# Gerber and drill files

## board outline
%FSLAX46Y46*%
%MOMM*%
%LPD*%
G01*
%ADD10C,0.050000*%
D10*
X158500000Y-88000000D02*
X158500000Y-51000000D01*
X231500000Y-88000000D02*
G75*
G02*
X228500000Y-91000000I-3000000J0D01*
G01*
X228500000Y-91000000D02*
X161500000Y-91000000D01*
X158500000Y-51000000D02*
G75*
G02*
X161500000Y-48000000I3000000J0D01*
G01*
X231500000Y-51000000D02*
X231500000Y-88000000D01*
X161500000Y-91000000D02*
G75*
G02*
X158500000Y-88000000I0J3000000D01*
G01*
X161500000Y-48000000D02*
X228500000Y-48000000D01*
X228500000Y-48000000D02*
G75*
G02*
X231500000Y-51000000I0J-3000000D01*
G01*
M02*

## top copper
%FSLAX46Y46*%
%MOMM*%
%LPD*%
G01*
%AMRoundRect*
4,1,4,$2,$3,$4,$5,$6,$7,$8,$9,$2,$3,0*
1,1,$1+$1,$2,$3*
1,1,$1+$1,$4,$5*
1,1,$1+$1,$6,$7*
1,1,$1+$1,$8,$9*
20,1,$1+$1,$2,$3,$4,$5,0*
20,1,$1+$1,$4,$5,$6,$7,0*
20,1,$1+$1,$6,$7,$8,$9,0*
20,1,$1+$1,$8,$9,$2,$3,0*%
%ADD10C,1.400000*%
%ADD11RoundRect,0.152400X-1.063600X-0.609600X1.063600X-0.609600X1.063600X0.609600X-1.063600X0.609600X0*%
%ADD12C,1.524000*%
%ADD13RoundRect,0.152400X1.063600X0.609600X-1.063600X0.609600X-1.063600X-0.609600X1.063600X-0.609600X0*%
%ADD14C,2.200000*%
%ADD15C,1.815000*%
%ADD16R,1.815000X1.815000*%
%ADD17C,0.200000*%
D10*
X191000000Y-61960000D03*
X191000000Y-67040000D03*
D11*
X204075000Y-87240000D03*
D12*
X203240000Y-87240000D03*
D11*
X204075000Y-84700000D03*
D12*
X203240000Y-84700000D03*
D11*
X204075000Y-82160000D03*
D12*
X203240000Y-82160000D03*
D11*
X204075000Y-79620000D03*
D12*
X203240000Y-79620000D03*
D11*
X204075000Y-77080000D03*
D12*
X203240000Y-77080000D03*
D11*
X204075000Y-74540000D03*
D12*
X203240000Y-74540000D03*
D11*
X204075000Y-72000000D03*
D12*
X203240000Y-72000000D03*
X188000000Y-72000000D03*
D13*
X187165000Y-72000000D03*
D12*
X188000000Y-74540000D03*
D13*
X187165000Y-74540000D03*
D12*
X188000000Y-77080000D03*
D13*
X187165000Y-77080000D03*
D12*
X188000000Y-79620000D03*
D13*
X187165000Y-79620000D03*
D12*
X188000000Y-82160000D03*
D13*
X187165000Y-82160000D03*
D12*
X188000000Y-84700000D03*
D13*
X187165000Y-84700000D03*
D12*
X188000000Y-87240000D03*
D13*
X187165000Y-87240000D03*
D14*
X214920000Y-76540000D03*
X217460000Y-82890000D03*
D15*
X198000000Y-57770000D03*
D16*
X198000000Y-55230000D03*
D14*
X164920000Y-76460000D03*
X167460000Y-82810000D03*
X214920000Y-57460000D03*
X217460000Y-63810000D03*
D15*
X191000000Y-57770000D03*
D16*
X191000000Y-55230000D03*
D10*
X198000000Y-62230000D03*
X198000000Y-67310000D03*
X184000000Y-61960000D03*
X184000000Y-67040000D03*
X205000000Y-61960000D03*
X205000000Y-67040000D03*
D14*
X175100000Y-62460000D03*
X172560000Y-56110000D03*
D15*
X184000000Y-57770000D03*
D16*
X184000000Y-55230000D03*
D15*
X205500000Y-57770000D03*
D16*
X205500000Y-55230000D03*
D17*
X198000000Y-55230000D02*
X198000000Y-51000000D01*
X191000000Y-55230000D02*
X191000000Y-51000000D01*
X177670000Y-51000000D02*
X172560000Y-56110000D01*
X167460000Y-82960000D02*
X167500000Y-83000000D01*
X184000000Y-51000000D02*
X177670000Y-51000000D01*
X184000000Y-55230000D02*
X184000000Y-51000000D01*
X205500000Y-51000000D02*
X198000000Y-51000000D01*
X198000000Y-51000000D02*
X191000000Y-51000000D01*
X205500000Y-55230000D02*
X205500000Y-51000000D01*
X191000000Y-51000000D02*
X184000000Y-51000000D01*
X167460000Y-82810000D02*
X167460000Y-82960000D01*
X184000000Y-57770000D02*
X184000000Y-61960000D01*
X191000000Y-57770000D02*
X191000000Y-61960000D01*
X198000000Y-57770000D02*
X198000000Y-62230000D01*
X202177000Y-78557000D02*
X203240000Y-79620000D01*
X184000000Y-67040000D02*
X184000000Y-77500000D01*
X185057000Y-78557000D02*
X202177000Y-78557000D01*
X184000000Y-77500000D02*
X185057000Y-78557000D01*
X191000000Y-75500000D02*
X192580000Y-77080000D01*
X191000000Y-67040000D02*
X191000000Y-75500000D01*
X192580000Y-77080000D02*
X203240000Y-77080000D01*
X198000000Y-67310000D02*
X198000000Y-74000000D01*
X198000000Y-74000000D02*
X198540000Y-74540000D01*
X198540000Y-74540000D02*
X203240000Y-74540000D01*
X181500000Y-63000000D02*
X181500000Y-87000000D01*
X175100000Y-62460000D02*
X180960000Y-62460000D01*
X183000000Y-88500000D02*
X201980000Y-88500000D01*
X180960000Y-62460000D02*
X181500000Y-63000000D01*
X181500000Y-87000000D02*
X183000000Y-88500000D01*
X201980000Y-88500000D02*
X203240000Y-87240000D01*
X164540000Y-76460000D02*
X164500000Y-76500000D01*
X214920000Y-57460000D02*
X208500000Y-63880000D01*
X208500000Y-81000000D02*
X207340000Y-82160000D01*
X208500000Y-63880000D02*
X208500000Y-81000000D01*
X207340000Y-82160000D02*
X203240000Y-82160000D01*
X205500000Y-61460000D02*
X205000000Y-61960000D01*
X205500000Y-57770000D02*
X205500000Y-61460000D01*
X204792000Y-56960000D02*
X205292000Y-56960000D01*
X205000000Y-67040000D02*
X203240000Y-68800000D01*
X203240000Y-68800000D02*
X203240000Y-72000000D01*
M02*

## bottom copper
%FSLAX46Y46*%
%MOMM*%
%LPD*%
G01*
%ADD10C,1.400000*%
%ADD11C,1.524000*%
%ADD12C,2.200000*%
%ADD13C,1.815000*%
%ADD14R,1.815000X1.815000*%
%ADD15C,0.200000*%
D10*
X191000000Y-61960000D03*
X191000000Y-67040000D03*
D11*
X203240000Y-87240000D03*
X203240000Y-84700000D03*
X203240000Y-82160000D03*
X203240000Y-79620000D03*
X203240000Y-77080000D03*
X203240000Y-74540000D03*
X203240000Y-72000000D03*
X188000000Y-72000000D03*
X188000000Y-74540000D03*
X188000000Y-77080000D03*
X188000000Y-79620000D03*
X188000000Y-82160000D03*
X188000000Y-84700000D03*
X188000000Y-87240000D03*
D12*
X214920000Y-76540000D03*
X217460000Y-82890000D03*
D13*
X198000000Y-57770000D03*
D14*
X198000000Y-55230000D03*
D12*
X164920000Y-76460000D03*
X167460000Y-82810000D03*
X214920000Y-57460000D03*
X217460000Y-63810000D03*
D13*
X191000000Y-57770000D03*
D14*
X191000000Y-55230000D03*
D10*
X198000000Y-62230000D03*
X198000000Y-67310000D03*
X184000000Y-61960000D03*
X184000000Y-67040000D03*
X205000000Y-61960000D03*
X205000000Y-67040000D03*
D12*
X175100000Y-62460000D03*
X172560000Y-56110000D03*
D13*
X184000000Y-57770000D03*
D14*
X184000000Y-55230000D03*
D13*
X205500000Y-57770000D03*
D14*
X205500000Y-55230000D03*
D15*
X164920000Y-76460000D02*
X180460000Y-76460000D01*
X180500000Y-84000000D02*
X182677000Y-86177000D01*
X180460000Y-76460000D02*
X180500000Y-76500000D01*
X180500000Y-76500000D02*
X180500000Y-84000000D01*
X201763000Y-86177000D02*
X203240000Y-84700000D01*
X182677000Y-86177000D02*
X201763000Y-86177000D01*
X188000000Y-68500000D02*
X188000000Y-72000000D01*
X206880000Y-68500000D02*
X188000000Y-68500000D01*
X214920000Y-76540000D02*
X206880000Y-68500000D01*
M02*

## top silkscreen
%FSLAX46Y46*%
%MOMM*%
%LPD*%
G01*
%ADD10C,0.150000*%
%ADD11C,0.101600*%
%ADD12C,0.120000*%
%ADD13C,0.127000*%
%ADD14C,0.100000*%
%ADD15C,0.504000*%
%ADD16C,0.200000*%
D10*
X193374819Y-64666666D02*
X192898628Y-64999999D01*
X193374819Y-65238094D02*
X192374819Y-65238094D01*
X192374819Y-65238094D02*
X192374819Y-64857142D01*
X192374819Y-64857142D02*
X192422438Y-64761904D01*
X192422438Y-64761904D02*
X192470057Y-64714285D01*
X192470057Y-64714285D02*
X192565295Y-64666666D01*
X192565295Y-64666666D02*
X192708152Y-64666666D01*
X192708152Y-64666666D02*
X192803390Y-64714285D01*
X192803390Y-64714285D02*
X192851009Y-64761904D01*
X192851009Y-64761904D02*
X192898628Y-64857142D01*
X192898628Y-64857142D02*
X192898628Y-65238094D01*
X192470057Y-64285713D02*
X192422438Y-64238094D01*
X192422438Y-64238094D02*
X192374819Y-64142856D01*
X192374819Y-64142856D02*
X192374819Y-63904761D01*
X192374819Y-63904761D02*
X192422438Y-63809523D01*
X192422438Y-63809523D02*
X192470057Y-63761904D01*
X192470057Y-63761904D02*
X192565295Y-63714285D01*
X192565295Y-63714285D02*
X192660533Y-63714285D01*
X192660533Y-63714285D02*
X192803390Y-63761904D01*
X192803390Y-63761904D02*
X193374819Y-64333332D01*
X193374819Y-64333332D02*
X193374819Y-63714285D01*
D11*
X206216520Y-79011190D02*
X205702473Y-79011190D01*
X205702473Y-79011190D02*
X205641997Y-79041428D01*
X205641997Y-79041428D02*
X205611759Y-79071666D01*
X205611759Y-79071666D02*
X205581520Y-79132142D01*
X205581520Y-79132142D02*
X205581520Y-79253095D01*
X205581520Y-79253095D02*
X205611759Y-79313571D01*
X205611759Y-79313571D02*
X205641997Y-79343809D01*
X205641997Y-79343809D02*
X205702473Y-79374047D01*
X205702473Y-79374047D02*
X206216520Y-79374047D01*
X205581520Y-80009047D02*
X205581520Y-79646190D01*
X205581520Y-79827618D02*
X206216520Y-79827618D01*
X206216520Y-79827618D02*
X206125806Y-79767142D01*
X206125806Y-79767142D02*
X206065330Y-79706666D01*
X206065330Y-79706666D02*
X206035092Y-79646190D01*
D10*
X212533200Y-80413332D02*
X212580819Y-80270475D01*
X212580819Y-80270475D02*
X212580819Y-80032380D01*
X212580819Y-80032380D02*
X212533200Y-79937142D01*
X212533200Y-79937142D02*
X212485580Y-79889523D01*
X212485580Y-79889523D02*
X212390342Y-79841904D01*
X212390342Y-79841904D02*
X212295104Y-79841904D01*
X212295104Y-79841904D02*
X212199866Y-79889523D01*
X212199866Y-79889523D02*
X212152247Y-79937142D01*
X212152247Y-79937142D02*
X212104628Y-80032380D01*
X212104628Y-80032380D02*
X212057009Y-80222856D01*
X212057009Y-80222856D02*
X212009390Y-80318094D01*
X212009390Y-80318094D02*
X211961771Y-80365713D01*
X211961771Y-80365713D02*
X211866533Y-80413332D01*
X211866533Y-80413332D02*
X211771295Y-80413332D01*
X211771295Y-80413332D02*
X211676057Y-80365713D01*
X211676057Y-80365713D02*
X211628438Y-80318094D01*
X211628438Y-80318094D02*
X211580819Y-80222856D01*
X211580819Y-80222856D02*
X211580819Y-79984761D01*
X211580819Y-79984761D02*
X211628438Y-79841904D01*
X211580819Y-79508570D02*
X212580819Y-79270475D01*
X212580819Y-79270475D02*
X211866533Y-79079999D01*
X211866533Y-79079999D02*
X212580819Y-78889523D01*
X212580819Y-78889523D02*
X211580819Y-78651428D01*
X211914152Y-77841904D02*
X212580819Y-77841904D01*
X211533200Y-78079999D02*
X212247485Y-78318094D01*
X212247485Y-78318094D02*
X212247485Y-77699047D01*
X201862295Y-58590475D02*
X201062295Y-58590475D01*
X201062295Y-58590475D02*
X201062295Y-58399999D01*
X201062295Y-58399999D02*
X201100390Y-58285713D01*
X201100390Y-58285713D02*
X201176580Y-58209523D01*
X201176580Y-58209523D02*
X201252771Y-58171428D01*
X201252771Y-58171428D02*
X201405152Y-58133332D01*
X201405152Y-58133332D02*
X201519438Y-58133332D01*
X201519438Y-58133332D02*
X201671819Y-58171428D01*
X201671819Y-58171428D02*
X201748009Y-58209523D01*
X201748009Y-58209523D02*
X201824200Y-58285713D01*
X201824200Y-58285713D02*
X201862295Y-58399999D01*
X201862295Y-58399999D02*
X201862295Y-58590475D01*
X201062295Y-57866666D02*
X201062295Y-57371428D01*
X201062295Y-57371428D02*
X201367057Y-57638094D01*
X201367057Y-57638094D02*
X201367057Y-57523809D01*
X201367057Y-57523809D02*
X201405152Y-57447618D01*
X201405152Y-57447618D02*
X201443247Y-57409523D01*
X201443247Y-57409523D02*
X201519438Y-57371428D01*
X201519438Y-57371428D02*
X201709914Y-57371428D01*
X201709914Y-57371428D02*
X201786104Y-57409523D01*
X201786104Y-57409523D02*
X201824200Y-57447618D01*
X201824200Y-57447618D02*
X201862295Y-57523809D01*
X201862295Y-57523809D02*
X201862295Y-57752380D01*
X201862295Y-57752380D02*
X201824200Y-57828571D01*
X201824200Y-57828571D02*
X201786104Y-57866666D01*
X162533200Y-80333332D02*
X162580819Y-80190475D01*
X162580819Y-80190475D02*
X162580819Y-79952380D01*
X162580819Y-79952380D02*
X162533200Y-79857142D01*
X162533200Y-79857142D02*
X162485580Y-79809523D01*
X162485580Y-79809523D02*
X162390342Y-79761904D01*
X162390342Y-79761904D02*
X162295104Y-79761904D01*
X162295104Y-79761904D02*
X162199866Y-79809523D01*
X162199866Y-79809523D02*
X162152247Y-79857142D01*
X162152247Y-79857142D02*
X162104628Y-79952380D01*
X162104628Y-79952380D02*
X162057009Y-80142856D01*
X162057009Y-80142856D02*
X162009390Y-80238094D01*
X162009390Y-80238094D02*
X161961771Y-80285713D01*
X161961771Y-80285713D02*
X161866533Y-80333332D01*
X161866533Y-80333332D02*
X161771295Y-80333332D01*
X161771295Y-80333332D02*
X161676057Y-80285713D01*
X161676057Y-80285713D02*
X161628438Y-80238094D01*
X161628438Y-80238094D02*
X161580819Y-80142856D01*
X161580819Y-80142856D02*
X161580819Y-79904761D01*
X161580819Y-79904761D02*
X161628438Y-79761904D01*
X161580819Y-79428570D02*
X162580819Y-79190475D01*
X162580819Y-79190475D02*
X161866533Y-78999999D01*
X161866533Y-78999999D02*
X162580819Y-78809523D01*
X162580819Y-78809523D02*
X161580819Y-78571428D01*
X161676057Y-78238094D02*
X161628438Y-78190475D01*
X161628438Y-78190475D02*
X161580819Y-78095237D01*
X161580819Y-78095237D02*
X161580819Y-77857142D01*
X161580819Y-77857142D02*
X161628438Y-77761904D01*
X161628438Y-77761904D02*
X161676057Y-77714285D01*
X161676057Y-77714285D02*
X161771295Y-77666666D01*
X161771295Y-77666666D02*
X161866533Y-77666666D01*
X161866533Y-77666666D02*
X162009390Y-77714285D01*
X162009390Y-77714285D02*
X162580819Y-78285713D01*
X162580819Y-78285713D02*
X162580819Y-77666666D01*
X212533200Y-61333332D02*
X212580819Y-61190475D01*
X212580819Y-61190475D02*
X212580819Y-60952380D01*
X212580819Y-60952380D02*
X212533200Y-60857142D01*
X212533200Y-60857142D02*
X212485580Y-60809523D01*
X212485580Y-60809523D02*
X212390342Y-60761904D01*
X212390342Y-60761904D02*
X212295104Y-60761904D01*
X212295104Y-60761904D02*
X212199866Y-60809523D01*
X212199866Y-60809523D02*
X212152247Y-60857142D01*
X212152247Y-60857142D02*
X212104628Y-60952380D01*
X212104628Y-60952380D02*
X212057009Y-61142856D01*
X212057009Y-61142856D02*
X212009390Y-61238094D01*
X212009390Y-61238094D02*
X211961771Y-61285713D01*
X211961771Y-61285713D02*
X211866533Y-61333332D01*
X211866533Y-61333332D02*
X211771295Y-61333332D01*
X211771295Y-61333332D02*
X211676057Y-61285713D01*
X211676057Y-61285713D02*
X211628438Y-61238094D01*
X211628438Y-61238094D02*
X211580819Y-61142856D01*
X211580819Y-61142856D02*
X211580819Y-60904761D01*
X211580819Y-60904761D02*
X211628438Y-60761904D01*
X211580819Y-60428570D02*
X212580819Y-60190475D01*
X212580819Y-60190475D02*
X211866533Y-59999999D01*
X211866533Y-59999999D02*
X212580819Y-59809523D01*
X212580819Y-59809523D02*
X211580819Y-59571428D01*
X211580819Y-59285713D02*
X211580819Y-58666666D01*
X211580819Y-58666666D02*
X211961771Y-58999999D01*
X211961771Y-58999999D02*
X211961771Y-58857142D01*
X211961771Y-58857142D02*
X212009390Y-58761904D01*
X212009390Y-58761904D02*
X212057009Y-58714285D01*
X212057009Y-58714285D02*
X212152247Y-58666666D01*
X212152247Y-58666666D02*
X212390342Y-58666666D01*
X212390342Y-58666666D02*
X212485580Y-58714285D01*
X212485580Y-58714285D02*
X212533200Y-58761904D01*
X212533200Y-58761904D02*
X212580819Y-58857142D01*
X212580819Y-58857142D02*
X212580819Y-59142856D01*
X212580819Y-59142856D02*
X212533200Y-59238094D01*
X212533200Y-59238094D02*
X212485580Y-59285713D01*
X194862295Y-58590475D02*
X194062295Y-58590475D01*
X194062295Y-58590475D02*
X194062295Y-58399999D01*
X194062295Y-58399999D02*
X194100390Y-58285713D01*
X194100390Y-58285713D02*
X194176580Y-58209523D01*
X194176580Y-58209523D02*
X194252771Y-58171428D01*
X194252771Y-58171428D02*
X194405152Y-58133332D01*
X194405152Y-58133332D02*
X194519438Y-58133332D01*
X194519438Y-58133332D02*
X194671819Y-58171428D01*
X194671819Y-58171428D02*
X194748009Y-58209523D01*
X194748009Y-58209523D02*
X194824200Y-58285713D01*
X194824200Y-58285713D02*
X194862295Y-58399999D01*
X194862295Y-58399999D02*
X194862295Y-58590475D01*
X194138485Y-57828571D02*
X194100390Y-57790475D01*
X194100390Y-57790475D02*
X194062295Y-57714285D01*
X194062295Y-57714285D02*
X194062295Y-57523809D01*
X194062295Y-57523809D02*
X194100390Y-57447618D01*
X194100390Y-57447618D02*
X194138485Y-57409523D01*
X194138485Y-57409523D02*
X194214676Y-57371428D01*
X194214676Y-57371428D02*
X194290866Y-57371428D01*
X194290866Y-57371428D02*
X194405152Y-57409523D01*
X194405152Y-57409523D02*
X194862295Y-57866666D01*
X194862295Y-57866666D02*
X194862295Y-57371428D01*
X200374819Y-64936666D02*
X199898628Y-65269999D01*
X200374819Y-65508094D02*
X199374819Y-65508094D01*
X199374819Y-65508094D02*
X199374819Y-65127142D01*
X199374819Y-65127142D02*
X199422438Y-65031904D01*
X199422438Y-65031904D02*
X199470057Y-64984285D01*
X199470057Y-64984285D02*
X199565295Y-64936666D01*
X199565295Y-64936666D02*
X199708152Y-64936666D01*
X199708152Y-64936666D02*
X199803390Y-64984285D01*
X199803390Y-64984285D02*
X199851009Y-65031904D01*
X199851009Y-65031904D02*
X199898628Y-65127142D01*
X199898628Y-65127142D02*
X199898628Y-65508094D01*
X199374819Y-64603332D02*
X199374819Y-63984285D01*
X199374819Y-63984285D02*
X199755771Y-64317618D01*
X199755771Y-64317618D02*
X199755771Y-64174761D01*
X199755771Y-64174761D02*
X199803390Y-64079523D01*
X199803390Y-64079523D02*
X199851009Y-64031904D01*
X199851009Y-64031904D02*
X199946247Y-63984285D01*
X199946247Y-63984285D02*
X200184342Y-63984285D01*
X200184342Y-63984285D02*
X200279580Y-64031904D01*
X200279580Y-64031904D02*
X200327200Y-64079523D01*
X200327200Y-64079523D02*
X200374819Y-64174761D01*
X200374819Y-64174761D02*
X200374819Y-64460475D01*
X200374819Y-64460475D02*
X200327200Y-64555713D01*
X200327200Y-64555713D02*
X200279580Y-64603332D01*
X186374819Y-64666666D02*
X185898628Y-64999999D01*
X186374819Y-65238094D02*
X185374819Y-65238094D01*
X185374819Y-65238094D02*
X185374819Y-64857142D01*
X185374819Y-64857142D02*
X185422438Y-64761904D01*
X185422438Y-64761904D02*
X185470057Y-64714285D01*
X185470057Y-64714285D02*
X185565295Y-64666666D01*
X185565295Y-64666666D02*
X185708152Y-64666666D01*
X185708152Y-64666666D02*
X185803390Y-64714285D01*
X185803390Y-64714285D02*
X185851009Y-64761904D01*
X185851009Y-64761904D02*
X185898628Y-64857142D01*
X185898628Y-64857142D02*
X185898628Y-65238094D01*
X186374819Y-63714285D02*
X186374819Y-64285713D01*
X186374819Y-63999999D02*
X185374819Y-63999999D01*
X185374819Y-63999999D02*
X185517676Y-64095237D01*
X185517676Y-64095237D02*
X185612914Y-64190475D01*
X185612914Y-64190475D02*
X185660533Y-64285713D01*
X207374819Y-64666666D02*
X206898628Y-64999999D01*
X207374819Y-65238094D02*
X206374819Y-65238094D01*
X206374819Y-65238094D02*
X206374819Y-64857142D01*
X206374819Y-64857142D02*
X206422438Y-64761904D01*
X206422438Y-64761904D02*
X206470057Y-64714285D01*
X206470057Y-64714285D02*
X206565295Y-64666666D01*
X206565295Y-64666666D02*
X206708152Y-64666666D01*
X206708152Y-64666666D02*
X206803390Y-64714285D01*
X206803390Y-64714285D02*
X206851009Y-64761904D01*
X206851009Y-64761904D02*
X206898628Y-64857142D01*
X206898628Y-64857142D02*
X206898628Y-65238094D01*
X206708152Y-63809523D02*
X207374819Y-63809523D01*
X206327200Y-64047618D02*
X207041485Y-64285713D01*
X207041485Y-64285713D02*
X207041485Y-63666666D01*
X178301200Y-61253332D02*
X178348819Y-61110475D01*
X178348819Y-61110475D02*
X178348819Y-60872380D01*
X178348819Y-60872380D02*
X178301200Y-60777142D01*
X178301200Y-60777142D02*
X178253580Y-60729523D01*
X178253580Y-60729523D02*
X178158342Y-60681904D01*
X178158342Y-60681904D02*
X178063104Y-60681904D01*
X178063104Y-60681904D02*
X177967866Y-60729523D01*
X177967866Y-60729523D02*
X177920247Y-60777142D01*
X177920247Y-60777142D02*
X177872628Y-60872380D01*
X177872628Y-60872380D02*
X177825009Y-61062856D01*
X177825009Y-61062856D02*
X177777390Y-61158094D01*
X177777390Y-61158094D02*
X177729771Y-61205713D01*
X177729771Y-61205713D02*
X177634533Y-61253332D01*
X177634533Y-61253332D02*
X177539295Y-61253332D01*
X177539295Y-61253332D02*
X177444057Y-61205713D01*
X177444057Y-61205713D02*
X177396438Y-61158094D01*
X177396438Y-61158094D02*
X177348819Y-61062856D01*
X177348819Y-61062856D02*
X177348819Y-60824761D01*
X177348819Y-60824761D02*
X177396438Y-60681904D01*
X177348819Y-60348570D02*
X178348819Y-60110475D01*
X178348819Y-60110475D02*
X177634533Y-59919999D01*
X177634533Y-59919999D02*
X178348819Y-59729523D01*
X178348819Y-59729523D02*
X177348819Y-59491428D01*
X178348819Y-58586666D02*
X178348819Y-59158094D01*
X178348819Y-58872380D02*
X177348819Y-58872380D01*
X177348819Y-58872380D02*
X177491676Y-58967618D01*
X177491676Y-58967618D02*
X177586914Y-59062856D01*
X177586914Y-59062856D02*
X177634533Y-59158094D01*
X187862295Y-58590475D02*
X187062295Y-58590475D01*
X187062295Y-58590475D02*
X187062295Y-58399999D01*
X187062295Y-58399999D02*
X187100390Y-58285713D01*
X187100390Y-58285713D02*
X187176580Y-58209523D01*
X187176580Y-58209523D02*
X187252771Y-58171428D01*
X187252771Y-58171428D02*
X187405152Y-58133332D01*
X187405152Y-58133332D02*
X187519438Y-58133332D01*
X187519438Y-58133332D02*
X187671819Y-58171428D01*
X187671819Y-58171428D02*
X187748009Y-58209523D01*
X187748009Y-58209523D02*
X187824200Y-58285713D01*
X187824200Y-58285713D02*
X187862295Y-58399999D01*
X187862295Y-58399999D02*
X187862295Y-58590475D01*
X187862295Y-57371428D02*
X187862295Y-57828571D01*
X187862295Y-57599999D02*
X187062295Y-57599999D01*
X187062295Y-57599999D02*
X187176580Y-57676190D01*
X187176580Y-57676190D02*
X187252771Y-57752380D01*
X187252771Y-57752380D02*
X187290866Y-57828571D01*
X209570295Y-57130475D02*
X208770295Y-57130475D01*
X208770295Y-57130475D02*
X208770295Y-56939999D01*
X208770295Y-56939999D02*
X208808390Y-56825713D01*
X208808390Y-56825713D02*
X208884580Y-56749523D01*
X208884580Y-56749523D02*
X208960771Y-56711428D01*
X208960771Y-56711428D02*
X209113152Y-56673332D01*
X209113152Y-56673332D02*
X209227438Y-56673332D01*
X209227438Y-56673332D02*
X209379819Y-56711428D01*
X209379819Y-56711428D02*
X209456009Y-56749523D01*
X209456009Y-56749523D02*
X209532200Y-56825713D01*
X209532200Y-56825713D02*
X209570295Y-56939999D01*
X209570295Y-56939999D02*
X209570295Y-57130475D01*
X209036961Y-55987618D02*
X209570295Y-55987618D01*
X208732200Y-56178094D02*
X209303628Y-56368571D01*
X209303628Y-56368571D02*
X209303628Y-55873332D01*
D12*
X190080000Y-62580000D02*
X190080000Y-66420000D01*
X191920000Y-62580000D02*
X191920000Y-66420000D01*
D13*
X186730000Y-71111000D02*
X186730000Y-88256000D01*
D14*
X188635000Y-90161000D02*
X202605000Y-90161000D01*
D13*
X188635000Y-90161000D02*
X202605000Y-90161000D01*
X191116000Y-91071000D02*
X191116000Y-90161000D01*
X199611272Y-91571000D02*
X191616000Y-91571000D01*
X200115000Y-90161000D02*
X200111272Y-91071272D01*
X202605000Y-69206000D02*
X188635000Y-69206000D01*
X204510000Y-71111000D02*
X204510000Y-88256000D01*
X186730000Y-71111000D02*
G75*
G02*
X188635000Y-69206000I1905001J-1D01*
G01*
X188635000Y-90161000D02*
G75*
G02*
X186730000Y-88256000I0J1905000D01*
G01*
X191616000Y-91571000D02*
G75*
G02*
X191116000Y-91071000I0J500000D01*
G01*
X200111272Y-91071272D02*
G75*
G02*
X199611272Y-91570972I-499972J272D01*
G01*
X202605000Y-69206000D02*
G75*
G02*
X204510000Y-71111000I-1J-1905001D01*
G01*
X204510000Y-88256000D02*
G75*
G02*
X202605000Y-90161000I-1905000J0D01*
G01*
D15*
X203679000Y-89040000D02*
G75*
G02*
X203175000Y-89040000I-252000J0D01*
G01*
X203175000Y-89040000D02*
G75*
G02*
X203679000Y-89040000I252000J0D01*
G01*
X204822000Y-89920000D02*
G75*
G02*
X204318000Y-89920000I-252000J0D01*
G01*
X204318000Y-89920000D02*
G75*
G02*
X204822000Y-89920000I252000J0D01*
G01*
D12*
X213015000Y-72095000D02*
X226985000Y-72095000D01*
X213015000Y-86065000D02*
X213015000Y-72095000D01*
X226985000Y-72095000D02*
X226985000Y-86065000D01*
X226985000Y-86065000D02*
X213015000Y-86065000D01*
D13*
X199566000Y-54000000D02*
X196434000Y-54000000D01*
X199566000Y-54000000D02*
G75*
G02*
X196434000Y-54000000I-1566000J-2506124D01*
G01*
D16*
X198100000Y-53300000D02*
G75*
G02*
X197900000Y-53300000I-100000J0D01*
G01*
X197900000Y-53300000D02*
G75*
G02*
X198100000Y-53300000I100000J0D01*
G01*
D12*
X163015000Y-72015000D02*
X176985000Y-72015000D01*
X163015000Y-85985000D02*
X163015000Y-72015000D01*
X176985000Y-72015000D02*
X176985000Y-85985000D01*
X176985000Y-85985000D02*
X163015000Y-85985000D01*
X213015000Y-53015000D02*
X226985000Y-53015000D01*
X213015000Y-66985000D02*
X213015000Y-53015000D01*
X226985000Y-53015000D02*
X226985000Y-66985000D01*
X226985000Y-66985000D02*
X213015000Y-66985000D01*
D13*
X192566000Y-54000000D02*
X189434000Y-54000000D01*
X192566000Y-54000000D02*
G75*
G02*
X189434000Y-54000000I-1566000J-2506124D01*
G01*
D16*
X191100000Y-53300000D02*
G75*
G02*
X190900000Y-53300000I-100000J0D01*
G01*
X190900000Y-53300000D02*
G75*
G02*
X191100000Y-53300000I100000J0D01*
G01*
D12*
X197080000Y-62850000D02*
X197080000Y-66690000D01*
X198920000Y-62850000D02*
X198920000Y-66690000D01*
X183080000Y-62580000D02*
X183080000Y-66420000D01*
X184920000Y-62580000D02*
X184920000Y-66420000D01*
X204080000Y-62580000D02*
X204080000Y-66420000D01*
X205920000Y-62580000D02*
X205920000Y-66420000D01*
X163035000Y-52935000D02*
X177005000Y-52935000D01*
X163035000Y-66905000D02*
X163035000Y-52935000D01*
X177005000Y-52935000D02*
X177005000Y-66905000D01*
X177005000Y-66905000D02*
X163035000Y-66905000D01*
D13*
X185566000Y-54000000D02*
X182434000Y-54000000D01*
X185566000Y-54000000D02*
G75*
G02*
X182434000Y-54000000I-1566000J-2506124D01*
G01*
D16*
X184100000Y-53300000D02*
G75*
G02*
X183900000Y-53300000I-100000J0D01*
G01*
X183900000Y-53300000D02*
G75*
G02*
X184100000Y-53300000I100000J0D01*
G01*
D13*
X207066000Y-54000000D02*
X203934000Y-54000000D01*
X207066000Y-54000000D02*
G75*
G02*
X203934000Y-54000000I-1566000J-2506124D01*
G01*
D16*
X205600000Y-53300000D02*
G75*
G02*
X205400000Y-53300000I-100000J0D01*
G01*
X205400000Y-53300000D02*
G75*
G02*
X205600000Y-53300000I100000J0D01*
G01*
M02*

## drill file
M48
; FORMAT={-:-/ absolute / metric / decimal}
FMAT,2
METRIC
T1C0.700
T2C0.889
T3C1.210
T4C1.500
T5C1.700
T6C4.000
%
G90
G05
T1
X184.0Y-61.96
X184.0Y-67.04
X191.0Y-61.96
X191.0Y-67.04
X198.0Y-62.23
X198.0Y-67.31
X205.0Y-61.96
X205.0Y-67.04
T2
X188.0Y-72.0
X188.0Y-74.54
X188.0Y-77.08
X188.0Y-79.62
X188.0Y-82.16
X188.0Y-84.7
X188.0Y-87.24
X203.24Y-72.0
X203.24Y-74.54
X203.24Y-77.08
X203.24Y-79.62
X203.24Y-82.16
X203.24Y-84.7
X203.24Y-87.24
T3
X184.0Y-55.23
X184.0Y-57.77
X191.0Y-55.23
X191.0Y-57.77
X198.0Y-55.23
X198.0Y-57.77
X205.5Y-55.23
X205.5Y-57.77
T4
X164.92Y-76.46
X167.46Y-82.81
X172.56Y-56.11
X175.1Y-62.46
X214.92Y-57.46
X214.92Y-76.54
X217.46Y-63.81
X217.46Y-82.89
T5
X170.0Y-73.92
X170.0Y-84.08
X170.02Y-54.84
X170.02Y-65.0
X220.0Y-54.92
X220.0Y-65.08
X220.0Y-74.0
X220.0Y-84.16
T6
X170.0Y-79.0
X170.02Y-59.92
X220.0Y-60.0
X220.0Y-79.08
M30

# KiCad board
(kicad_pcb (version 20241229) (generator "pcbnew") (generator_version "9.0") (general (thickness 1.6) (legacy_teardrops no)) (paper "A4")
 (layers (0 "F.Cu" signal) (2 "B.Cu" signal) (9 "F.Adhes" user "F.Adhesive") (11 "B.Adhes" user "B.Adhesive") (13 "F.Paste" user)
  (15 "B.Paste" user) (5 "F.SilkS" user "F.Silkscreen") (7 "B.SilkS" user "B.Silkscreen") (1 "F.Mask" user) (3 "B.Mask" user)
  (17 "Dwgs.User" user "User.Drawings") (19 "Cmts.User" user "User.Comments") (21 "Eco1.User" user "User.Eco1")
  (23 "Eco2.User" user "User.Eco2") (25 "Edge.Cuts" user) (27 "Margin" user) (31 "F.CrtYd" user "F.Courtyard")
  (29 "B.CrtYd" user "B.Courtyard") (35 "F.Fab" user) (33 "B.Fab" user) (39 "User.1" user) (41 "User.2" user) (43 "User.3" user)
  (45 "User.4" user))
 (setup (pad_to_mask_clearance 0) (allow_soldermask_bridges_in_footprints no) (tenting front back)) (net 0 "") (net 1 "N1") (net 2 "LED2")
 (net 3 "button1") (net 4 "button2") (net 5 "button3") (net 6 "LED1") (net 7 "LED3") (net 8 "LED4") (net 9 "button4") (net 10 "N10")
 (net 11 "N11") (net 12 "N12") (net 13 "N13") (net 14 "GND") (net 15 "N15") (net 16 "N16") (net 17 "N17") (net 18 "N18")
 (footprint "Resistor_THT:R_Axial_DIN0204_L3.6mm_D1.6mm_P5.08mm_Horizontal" (layer "F.Cu") (at 191 61.96 -90)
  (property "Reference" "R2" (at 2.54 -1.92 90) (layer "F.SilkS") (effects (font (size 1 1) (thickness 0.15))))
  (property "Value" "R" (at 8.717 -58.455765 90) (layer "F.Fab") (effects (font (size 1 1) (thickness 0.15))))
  (fp_line (start 0.62 0.92) (end 4.46 0.92) (stroke (width 0.12) (type solid)) (layer "F.SilkS"))
  (fp_line (start 0.62 -0.92) (end 4.46 -0.92) (stroke (width 0.12) (type solid)) (layer "F.SilkS"))
  (pad "1" thru_hole circle (at 0 0 270) (size 1.4 1.4) (drill 0.7) (layers "*.Cu" "*.Mask") (remove_unused_layers no) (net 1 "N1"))
  (pad "2" thru_hole circle (at 5.08 0 270) (size 1.4 1.4) (drill 0.7) (layers "*.Cu" "*.Mask") (remove_unused_layers no) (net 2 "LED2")))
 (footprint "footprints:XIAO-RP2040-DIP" (layer "F.Cu") (at 195.62 79.62 -90)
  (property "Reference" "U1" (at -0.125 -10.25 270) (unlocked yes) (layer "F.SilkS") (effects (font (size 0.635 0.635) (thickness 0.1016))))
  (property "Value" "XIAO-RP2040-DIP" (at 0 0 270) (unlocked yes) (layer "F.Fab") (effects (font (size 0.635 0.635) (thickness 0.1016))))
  (fp_line (start -8.509 8.89) (end 8.636 8.89) (stroke (width 0.127) (type solid)) (layer "F.SilkS"))
  (fp_line (start 10.541 6.985) (end 10.541 -6.985) (stroke (width 0.1) (type solid)) (layer "F.SilkS"))
  (fp_line (start 10.541 6.985) (end 10.541 -6.985) (stroke (width 0.127) (type solid)) (layer "F.SilkS"))
  (fp_line (start 11.451 4.504) (end 10.541 4.504) (stroke (width 0.127) (type solid)) (layer "F.SilkS"))
  (fp_line (start 11.951 -3.991272) (end 11.951 4.004) (stroke (width 0.127) (type solid)) (layer "F.SilkS"))
  (fp_line (start 10.541 -4.495) (end 11.451272 -4.491272) (stroke (width 0.127) (type solid)) (layer "F.SilkS"))
  (fp_line (start -10.414 -6.985) (end -10.414 6.985) (stroke (width 0.127) (type solid)) (layer "F.SilkS"))
  (fp_line (start -8.509 -8.89) (end 8.636 -8.89) (stroke (width 0.127) (type solid)) (layer "F.SilkS"))
  (fp_arc (start -8.509 8.89) (mid -9.856038 8.332038) (end -10.414 6.985) (stroke (width 0.127) (type solid)) (layer "F.SilkS"))
  (fp_arc (start 10.541 6.985) (mid 9.983038 8.332038) (end 8.636 8.89) (stroke (width 0.127) (type solid)) (layer "F.SilkS"))
  (fp_arc (start 11.951 4.004) (mid 11.804553 4.357553) (end 11.451 4.504) (stroke (width 0.127) (type default)) (layer "F.SilkS"))
  (fp_arc (start 11.451272 -4.491272) (mid 11.804644 -4.344724) (end 11.951 -3.991272) (stroke (width 0.127) (type default))
   (layer "F.SilkS"))
  (fp_arc (start -10.414 -6.985) (mid -9.856038 -8.332038) (end -8.509 -8.89) (stroke (width 0.127) (type solid)) (layer "F.SilkS"))
  (fp_arc (start 8.636 -8.89) (mid 9.983038 -8.332038) (end 10.541 -6.985) (stroke (width 0.127) (type solid)) (layer "F.SilkS"))
  (fp_circle (center 9.42 -7.807) (end 9.674 -7.807) (stroke (width 0.5) (type solid)) (fill yes) (layer "F.SilkS"))
  (fp_circle (center 10.3 -8.95) (end 10.554 -8.95) (stroke (width 0.5) (type solid)) (fill yes) (layer "F.SilkS"))
  (pad "1" smd roundrect (at 7.62 -8.455) (size 2.432 1.524) (layers "F.Cu" "F.Mask") (roundrect_rratio 0.1) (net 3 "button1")
   (thermal_bridge_angle 45))
  (pad "1" thru_hole circle (at 7.62 -7.62) (size 1.524 1.524) (drill 0.889) (layers "*.Cu" "*.Mask") (remove_unused_layers no)
   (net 3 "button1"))
  (pad "2" smd roundrect (at 5.08 -8.455) (size 2.432 1.524) (layers "F.Cu" "F.Mask") (roundrect_rratio 0.1) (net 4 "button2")
   (thermal_bridge_angle 45))
  (pad "2" thru_hole circle (at 5.08 -7.62) (size 1.524 1.524) (drill 0.889) (layers "*.Cu" "*.Mask") (remove_unused_layers no)
   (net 4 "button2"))
  (pad "3" smd roundrect (at 2.54 -8.455) (size 2.432 1.524) (layers "F.Cu" "F.Mask") (roundrect_rratio 0.1) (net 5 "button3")
   (thermal_bridge_angle 45))
  (pad "3" thru_hole circle (at 2.54 -7.62) (size 1.524 1.524) (drill 0.889) (layers "*.Cu" "*.Mask") (remove_unused_layers no)
   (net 5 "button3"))
  (pad "4" smd roundrect (at 0 -8.455) (size 2.432 1.524) (layers "F.Cu" "F.Mask") (roundrect_rratio 0.1) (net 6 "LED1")
   (thermal_bridge_angle 45))
  (pad "4" thru_hole circle (at 0 -7.62) (size 1.524 1.524) (drill 0.889) (layers "*.Cu" "*.Mask") (remove_unused_layers no) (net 6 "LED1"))
  (pad "5" smd roundrect (at -2.54 -8.455) (size 2.432 1.524) (layers "F.Cu" "F.Mask") (roundrect_rratio 0.1) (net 2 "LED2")
   (thermal_bridge_angle 45))
  (pad "5" thru_hole circle (at -2.54 -7.62) (size 1.524 1.524) (drill 0.889) (layers "*.Cu" "*.Mask") (remove_unused_layers no)
   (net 2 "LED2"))
  (pad "6" smd roundrect (at -5.08 -8.455) (size 2.432 1.524) (layers "F.Cu" "F.Mask") (roundrect_rratio 0.1) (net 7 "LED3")
   (thermal_bridge_angle 45))
  (pad "6" thru_hole circle (at -5.08 -7.62) (size 1.524 1.524) (drill 0.889) (layers "*.Cu" "*.Mask") (remove_unused_layers no)
   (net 7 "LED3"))
  (pad "7" smd roundrect (at -7.62 -8.455) (size 2.432 1.524) (layers "F.Cu" "F.Mask") (roundrect_rratio 0.1) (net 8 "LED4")
   (thermal_bridge_angle 45))
  (pad "7" thru_hole circle (at -7.62 -7.62) (size 1.524 1.524) (drill 0.889) (layers "*.Cu" "*.Mask") (remove_unused_layers no)
   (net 8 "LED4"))
  (pad "8" thru_hole circle (at -7.62 7.62 180) (size 1.524 1.524) (drill 0.889) (layers "*.Cu" "*.Mask") (remove_unused_layers no)
   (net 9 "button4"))
  (pad "8" smd roundrect (at -7.62 8.455 180) (size 2.432 1.524) (layers "F.Cu" "F.Mask") (roundrect_rratio 0.1) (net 9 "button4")
   (thermal_bridge_angle 45))
  (pad "9" thru_hole circle (at -5.08 7.62 180) (size 1.524 1.524) (drill 0.889) (layers "*.Cu" "*.Mask") (remove_unused_layers no)
   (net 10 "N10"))
  (pad "9" smd roundrect (at -5.08 8.455 180) (size 2.432 1.524) (layers "F.Cu" "F.Mask") (roundrect_rratio 0.1) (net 10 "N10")
   (thermal_bridge_angle 45))
  (pad "10" thru_hole circle (at -2.54 7.62 180) (size 1.524 1.524) (drill 0.889) (layers "*.Cu" "*.Mask") (remove_unused_layers no)
   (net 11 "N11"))
  (pad "10" smd roundrect (at -2.54 8.455 180) (size 2.432 1.524) (layers "F.Cu" "F.Mask") (roundrect_rratio 0.1) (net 11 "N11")
   (thermal_bridge_angle 45))
  (pad "11" thru_hole circle (at 0 7.62 180) (size 1.524 1.524) (drill 0.889) (layers "*.Cu" "*.Mask") (remove_unused_layers no)
   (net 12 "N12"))
  (pad "11" smd roundrect (at 0 8.455 180) (size 2.432 1.524) (layers "F.Cu" "F.Mask") (roundrect_rratio 0.1) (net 12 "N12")
   (thermal_bridge_angle 45))
  (pad "12" thru_hole circle (at 2.54 7.62 180) (size 1.524 1.524) (drill 0.889) (layers "*.Cu" "*.Mask") (remove_unused_layers no)
   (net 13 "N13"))
  (pad "12" smd roundrect (at 2.54 8.455 180) (size 2.432 1.524) (layers "F.Cu" "F.Mask") (roundrect_rratio 0.1) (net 13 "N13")
   (thermal_bridge_angle 45))
  (pad "13" thru_hole circle (at 5.08 7.62 180) (size 1.524 1.524) (drill 0.889) (layers "*.Cu" "*.Mask") (remove_unused_layers no)
   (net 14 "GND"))
  (pad "13" smd roundrect (at 5.08 8.455 180) (size 2.432 1.524) (layers "F.Cu" "F.Mask") (roundrect_rratio 0.1) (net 14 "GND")
   (thermal_bridge_angle 45))
  (pad "14" thru_hole circle (at 7.62 7.62 180) (size 1.524 1.524) (drill 0.889) (layers "*.Cu" "*.Mask") (remove_unused_layers no)
   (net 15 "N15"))
  (pad "14" smd roundrect (at 7.62 8.455 180) (size 2.432 1.524) (layers "F.Cu" "F.Mask") (roundrect_rratio 0.1) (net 15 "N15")
   (thermal_bridge_angle 45)))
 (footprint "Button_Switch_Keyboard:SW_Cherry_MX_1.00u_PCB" (layer "F.Cu") (at 214.92 76.54 90)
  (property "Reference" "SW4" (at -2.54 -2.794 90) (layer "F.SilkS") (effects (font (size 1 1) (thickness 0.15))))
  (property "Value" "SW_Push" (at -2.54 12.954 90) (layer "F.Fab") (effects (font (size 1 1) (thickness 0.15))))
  (fp_line (start 4.445 -1.905) (end 4.445 12.065) (stroke (width 0.12) (type solid)) (layer "F.SilkS"))
  (fp_line (start -9.525 -1.905) (end 4.445 -1.905) (stroke (width 0.12) (type solid)) (layer "F.SilkS"))
  (fp_line (start 4.445 12.065) (end -9.525 12.065) (stroke (width 0.12) (type solid)) (layer "F.SilkS"))
  (fp_line (start -9.525 12.065) (end -9.525 -1.905) (stroke (width 0.12) (type solid)) (layer "F.SilkS"))
  (pad "" np_thru_hole circle (at -7.62 5.08 90) (size 1.7 1.7) (drill 1.7) (layers "*.Cu" "*.Mask"))
  (pad "" np_thru_hole circle (at -2.54 5.08 90) (size 4 4) (drill 4) (layers "*.Cu" "*.Mask"))
  (pad "" np_thru_hole circle (at 2.54 5.08 90) (size 1.7 1.7) (drill 1.7) (layers "*.Cu" "*.Mask"))
  (pad "1" thru_hole circle (at 0 0 90) (size 2.2 2.2) (drill 1.5) (layers "*.Cu" "*.Mask") (remove_unused_layers no) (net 9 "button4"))
  (pad "2" thru_hole circle (at -6.35 2.54 90) (size 2.2 2.2) (drill 1.5) (layers "*.Cu" "*.Mask") (remove_unused_layers no) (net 14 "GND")))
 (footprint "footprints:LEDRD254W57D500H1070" (layer "F.Cu") (at 198 56.5 -90)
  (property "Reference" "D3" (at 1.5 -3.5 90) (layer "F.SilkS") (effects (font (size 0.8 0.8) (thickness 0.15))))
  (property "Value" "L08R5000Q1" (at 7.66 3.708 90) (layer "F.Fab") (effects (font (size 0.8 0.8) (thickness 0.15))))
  (fp_line (start -2.5 -1.566) (end -2.5 1.566) (stroke (width 0.127) (type solid)) (layer "F.SilkS"))
  (fp_arc (start -2.5 -1.566) (mid 2.961291 0) (end -2.5 1.566) (stroke (width 0.127) (type solid)) (layer "F.SilkS"))
  (fp_circle (center -3.2 0) (end -3.1 0) (stroke (width 0.2) (type solid)) (fill no) (layer "F.SilkS"))
  (pad "A" thru_hole circle (at 1.27 0 270) (size 1.815 1.815) (drill 1.21) (layers "*.Cu" "*.Mask") (remove_unused_layers no)
   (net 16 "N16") (solder_mask_margin 0.102))
  (pad "C" thru_hole rect (at -1.27 0 270) (size 1.815 1.815) (drill 1.21) (layers "*.Cu" "*.Mask") (remove_unused_layers no) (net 14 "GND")
   (solder_mask_margin 0.102)))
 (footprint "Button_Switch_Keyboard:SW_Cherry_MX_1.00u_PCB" (layer "F.Cu") (at 164.92 76.46 90)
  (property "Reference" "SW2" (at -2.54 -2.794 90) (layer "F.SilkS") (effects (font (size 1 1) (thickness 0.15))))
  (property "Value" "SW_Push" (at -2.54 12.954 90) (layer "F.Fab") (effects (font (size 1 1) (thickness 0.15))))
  (fp_line (start 4.445 -1.905) (end 4.445 12.065) (stroke (width 0.12) (type solid)) (layer "F.SilkS"))
  (fp_line (start -9.525 -1.905) (end 4.445 -1.905) (stroke (width 0.12) (type solid)) (layer "F.SilkS"))
  (fp_line (start 4.445 12.065) (end -9.525 12.065) (stroke (width 0.12) (type solid)) (layer "F.SilkS"))
  (fp_line (start -9.525 12.065) (end -9.525 -1.905) (stroke (width 0.12) (type solid)) (layer "F.SilkS"))
  (pad "" np_thru_hole circle (at -7.62 5.08 90) (size 1.7 1.7) (drill 1.7) (layers "*.Cu" "*.Mask"))
  (pad "" np_thru_hole circle (at -2.54 5.08 90) (size 4 4) (drill 4) (layers "*.Cu" "*.Mask"))
  (pad "" np_thru_hole circle (at 2.54 5.08 90) (size 1.7 1.7) (drill 1.7) (layers "*.Cu" "*.Mask"))
  (pad "1" thru_hole circle (at 0 0 90) (size 2.2 2.2) (drill 1.5) (layers "*.Cu" "*.Mask") (remove_unused_layers no) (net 4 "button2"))
  (pad "2" thru_hole circle (at -6.35 2.54 90) (size 2.2 2.2) (drill 1.5) (layers "*.Cu" "*.Mask") (remove_unused_layers no) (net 14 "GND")))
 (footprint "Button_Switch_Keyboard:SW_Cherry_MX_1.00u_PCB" (layer "F.Cu") (at 214.92 57.46 90)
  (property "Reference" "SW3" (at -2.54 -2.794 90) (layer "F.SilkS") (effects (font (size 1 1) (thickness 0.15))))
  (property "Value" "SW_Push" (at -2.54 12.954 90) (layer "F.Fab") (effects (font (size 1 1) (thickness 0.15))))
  (fp_line (start 4.445 -1.905) (end 4.445 12.065) (stroke (width 0.12) (type solid)) (layer "F.SilkS"))
  (fp_line (start -9.525 -1.905) (end 4.445 -1.905) (stroke (width 0.12) (type solid)) (layer "F.SilkS"))
  (fp_line (start 4.445 12.065) (end -9.525 12.065) (stroke (width 0.12) (type solid)) (layer "F.SilkS"))
  (fp_line (start -9.525 12.065) (end -9.525 -1.905) (stroke (width 0.12) (type solid)) (layer "F.SilkS"))
  (pad "" np_thru_hole circle (at -7.62 5.08 90) (size 1.7 1.7) (drill 1.7) (layers "*.Cu" "*.Mask"))
  (pad "" np_thru_hole circle (at -2.54 5.08 90) (size 4 4) (drill 4) (layers "*.Cu" "*.Mask"))
  (pad "" np_thru_hole circle (at 2.54 5.08 90) (size 1.7 1.7) (drill 1.7) (layers "*.Cu" "*.Mask"))
  (pad "1" thru_hole circle (at 0 0 90) (size 2.2 2.2) (drill 1.5) (layers "*.Cu" "*.Mask") (remove_unused_layers no) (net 5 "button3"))
  (pad "2" thru_hole circle (at -6.35 2.54 90) (size 2.2 2.2) (drill 1.5) (layers "*.Cu" "*.Mask") (remove_unused_layers no) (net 14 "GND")))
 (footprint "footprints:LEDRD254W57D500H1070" (layer "F.Cu") (at 191 56.5 -90)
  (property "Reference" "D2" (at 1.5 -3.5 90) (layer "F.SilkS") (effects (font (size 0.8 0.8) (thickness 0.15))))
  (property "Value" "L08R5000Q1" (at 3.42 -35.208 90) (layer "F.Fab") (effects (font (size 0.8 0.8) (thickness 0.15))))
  (fp_line (start -2.5 -1.566) (end -2.5 1.566) (stroke (width 0.127) (type solid)) (layer "F.SilkS"))
  (fp_arc (start -2.5 -1.566) (mid 2.961291 0) (end -2.5 1.566) (stroke (width 0.127) (type solid)) (layer "F.SilkS"))
  (fp_circle (center -3.2 0) (end -3.1 0) (stroke (width 0.2) (type solid)) (fill no) (layer "F.SilkS"))
  (pad "A" thru_hole circle (at 1.27 0 270) (size 1.815 1.815) (drill 1.21) (layers "*.Cu" "*.Mask") (remove_unused_layers no) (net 1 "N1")
   (solder_mask_margin 0.102))
  (pad "C" thru_hole rect (at -1.27 0 270) (size 1.815 1.815) (drill 1.21) (layers "*.Cu" "*.Mask") (remove_unused_layers no) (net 14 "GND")
   (solder_mask_margin 0.102)))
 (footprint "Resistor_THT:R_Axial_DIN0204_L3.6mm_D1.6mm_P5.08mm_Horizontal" (layer "F.Cu") (at 198 62.23 -90)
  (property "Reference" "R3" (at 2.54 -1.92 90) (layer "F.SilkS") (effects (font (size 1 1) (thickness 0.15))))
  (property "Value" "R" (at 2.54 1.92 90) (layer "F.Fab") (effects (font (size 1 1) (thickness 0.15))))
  (fp_line (start 0.62 0.92) (end 4.46 0.92) (stroke (width 0.12) (type solid)) (layer "F.SilkS"))
  (fp_line (start 0.62 -0.92) (end 4.46 -0.92) (stroke (width 0.12) (type solid)) (layer "F.SilkS"))
  (pad "1" thru_hole circle (at 0 0 270) (size 1.4 1.4) (drill 0.7) (layers "*.Cu" "*.Mask") (remove_unused_layers no) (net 16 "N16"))
  (pad "2" thru_hole circle (at 5.08 0 270) (size 1.4 1.4) (drill 0.7) (layers "*.Cu" "*.Mask") (remove_unused_layers no) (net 7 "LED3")))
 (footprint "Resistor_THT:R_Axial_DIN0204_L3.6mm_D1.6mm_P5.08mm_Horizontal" (layer "F.Cu") (at 184 61.96 -90)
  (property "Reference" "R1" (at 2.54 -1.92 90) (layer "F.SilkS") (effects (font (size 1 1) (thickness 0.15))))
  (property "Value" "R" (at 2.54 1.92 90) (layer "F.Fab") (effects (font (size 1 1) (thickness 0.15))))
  (fp_line (start 0.62 0.92) (end 4.46 0.92) (stroke (width 0.12) (type solid)) (layer "F.SilkS"))
  (fp_line (start 0.62 -0.92) (end 4.46 -0.92) (stroke (width 0.12) (type solid)) (layer "F.SilkS"))
  (pad "1" thru_hole circle (at 0 0 270) (size 1.4 1.4) (drill 0.7) (layers "*.Cu" "*.Mask") (remove_unused_layers no) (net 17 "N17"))
  (pad "2" thru_hole circle (at 5.08 0 270) (size 1.4 1.4) (drill 0.7) (layers "*.Cu" "*.Mask") (remove_unused_layers no) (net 6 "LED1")))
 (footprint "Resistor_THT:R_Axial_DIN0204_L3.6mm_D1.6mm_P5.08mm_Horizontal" (layer "F.Cu") (at 205 61.96 -90)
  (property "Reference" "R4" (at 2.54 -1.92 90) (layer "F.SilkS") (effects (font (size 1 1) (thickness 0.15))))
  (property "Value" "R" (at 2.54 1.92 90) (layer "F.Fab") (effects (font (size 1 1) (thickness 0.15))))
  (fp_line (start 0.62 0.92) (end 4.46 0.92) (stroke (width 0.12) (type solid)) (layer "F.SilkS"))
  (fp_line (start 0.62 -0.92) (end 4.46 -0.92) (stroke (width 0.12) (type solid)) (layer "F.SilkS"))
  (pad "1" thru_hole circle (at 0 0 270) (size 1.4 1.4) (drill 0.7) (layers "*.Cu" "*.Mask") (remove_unused_layers no) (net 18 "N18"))
  (pad "2" thru_hole circle (at 5.08 0 270) (size 1.4 1.4) (drill 0.7) (layers "*.Cu" "*.Mask") (remove_unused_layers no) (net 8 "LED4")))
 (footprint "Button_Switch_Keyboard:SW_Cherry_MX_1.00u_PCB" (layer "F.Cu") (at 175.1 62.46 -90)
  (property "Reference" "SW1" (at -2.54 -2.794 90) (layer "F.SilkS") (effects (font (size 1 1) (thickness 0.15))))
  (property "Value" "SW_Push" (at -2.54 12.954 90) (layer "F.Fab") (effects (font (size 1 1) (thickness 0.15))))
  (fp_line (start -9.525 12.065) (end -9.525 -1.905) (stroke (width 0.12) (type solid)) (layer "F.SilkS"))
  (fp_line (start 4.445 12.065) (end -9.525 12.065) (stroke (width 0.12) (type solid)) (layer "F.SilkS"))
  (fp_line (start -9.525 -1.905) (end 4.445 -1.905) (stroke (width 0.12) (type solid)) (layer "F.SilkS"))
  (fp_line (start 4.445 -1.905) (end 4.445 12.065) (stroke (width 0.12) (type solid)) (layer "F.SilkS"))
  (pad "" np_thru_hole circle (at -7.62 5.08 270) (size 1.7 1.7) (drill 1.7) (layers "*.Cu" "*.Mask"))
  (pad "" np_thru_hole circle (at -2.54 5.08 270) (size 4 4) (drill 4) (layers "*.Cu" "*.Mask"))
  (pad "" np_thru_hole circle (at 2.54 5.08 270) (size 1.7 1.7) (drill 1.7) (layers "*.Cu" "*.Mask"))
  (pad "1" thru_hole circle (at 0 0 270) (size 2.2 2.2) (drill 1.5) (layers "*.Cu" "*.Mask") (remove_unused_layers no) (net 3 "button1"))
  (pad "2" thru_hole circle (at -6.35 2.54 270) (size 2.2 2.2) (drill 1.5) (layers "*.Cu" "*.Mask") (remove_unused_layers no) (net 14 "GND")))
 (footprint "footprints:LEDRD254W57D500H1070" (layer "F.Cu") (at 184 56.5 -90)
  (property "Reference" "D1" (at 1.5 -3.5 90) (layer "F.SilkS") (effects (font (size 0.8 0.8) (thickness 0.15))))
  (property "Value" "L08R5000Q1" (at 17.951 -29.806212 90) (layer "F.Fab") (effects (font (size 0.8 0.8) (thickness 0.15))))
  (fp_line (start -2.5 -1.566) (end -2.5 1.566) (stroke (width 0.127) (type solid)) (layer "F.SilkS"))
  (fp_arc (start -2.5 -1.566) (mid 2.961291 0) (end -2.5 1.566) (stroke (width 0.127) (type solid)) (layer "F.SilkS"))
  (fp_circle (center -3.2 0) (end -3.1 0) (stroke (width 0.2) (type solid)) (fill no) (layer "F.SilkS"))
  (pad "A" thru_hole circle (at 1.27 0 270) (size 1.815 1.815) (drill 1.21) (layers "*.Cu" "*.Mask") (remove_unused_layers no)
   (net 17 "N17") (solder_mask_margin 0.102))
  (pad "C" thru_hole rect (at -1.27 0 270) (size 1.815 1.815) (drill 1.21) (layers "*.Cu" "*.Mask") (remove_unused_layers no) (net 14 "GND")
   (solder_mask_margin 0.102)))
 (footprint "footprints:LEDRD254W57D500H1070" (layer "F.Cu") (at 205.5 56.5 -90)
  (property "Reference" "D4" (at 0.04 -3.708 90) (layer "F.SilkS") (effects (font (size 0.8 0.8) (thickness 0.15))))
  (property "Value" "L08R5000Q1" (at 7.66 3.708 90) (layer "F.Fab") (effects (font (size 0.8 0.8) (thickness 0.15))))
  (fp_line (start -2.5 -1.566) (end -2.5 1.566) (stroke (width 0.127) (type solid)) (layer "F.SilkS"))
  (fp_arc (start -2.5 -1.566) (mid 2.961291 0) (end -2.5 1.566) (stroke (width 0.127) (type solid)) (layer "F.SilkS"))
  (fp_circle (center -3.2 0) (end -3.1 0) (stroke (width 0.2) (type solid)) (fill no) (layer "F.SilkS"))
  (pad "A" thru_hole circle (at 1.27 0 270) (size 1.815 1.815) (drill 1.21) (layers "*.Cu" "*.Mask") (remove_unused_layers no)
   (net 18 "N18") (solder_mask_margin 0.102))
  (pad "C" thru_hole rect (at -1.27 0 270) (size 1.815 1.815) (drill 1.21) (layers "*.Cu" "*.Mask") (remove_unused_layers no) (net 14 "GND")
   (solder_mask_margin 0.102)))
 (gr_line (start 158.5 88) (end 158.5 51) (stroke (width 0.05) (type default)) (layer "Edge.Cuts"))
 (gr_arc (start 231.5 88) (mid 230.62132 90.12132) (end 228.5 91) (stroke (width 0.05) (type default)) (layer "Edge.Cuts"))
 (gr_line (start 228.5 91) (end 161.5 91) (stroke (width 0.05) (type default)) (layer "Edge.Cuts"))
 (gr_arc (start 158.5 51) (mid 159.37868 48.87868) (end 161.5 48) (stroke (width 0.05) (type default)) (layer "Edge.Cuts"))
 (gr_line (start 231.5 51) (end 231.5 88) (stroke (width 0.05) (type default)) (layer "Edge.Cuts"))
 (gr_arc (start 161.5 91) (mid 159.37868 90.12132) (end 158.5 88) (stroke (width 0.05) (type default)) (layer "Edge.Cuts"))
 (gr_line (start 161.5 48) (end 228.5 48) (stroke (width 0.05) (type default)) (layer "Edge.Cuts"))
 (gr_arc (start 228.5 48) (mid 230.62132 48.87868) (end 231.5 51) (stroke (width 0.05) (type default)) (layer "Edge.Cuts"))
 (segment (start 198 55.23) (end 198 51) (width 0.2) (layer "F.Cu") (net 14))
 (segment (start 191 55.23) (end 191 51) (width 0.2) (layer "F.Cu") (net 14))
 (segment (start 177.67 51) (end 172.56 56.11) (width 0.2) (layer "F.Cu") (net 14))
 (segment (start 167.46 82.96) (end 167.5 83) (width 0.2) (layer "F.Cu") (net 14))
 (segment (start 184 51) (end 177.67 51) (width 0.2) (layer "F.Cu") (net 14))
 (segment (start 184 55.23) (end 184 51) (width 0.2) (layer "F.Cu") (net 14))
 (segment (start 205.5 51) (end 198 51) (width 0.2) (layer "F.Cu") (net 14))
 (segment (start 198 51) (end 191 51) (width 0.2) (layer "F.Cu") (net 14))
 (segment (start 205.5 55.23) (end 205.5 51) (width 0.2) (layer "F.Cu") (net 14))
 (segment (start 191 51) (end 184 51) (width 0.2) (layer "F.Cu") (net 14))
 (segment (start 167.46 82.81) (end 167.46 82.96) (width 0.2) (layer "F.Cu") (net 14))
 (segment (start 184 57.77) (end 184 61.96) (width 0.2) (layer "F.Cu") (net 17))
 (segment (start 191 57.77) (end 191 61.96) (width 0.2) (layer "F.Cu") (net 1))
 (segment (start 198 57.77) (end 198 62.23) (width 0.2) (layer "F.Cu") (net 16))
 (segment (start 202.177 78.557) (end 203.24 79.62) (width 0.2) (layer "F.Cu") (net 6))
 (segment (start 184 67.04) (end 184 77.5) (width 0.2) (layer "F.Cu") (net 6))
 (segment (start 185.057 78.557) (end 202.177 78.557) (width 0.2) (layer "F.Cu") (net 6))
 (segment (start 184 77.5) (end 185.057 78.557) (width 0.2) (layer "F.Cu") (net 6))
 (segment (start 191 75.5) (end 192.58 77.08) (width 0.2) (layer "F.Cu") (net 2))
 (segment (start 191 67.04) (end 191 75.5) (width 0.2) (layer "F.Cu") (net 2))
 (segment (start 192.58 77.08) (end 203.24 77.08) (width 0.2) (layer "F.Cu") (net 2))
 (segment (start 198 67.31) (end 198 74) (width 0.2) (layer "F.Cu") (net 7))
 (segment (start 198 74) (end 198.54 74.54) (width 0.2) (layer "F.Cu") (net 7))
 (segment (start 198.54 74.54) (end 203.24 74.54) (width 0.2) (layer "F.Cu") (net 7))
 (segment (start 181.5 63) (end 181.5 87) (width 0.2) (layer "F.Cu") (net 3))
 (segment (start 175.1 62.46) (end 180.96 62.46) (width 0.2) (layer "F.Cu") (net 3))
 (segment (start 183 88.5) (end 201.98 88.5) (width 0.2) (layer "F.Cu") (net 3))
 (segment (start 180.96 62.46) (end 181.5 63) (width 0.2) (layer "F.Cu") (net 3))
 (segment (start 181.5 87) (end 183 88.5) (width 0.2) (layer "F.Cu") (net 3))
 (segment (start 201.98 88.5) (end 203.24 87.24) (width 0.2) (layer "F.Cu") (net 3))
 (segment (start 164.54 76.46) (end 164.5 76.5) (width 0.2) (layer "F.Cu") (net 4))
 (segment (start 164.92 76.46) (end 180.46 76.46) (width 0.2) (layer "B.Cu") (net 4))
 (segment (start 180.5 84) (end 182.677 86.177) (width 0.2) (layer "B.Cu") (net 4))
 (segment (start 180.46 76.46) (end 180.5 76.5) (width 0.2) (layer "B.Cu") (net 4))
 (segment (start 180.5 76.5) (end 180.5 84) (width 0.2) (layer "B.Cu") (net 4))
 (segment (start 201.763 86.177) (end 203.24 84.7) (width 0.2) (layer "B.Cu") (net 4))
 (segment (start 182.677 86.177) (end 201.763 86.177) (width 0.2) (layer "B.Cu") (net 4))
 (segment (start 214.92 57.46) (end 208.5 63.88) (width 0.2) (layer "F.Cu") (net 5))
 (segment (start 208.5 81) (end 207.34 82.16) (width 0.2) (layer "F.Cu") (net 5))
 (segment (start 208.5 63.88) (end 208.5 81) (width 0.2) (layer "F.Cu") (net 5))
 (segment (start 207.34 82.16) (end 203.24 82.16) (width 0.2) (layer "F.Cu") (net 5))
 (segment (start 205.5 61.46) (end 205 61.96) (width 0.2) (layer "F.Cu") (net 18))
 (segment (start 205.5 57.77) (end 205.5 61.46) (width 0.2) (layer "F.Cu") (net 18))
 (segment (start 204.792 56.96) (end 205.292 56.96) (width 0.2) (layer "F.Cu") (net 18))
 (segment (start 205 67.04) (end 203.24 68.8) (width 0.2) (layer "F.Cu") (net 8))
 (segment (start 203.24 68.8) (end 203.24 72) (width 0.2) (layer "F.Cu") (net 8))
 (segment (start 188 68.5) (end 188 72) (width 0.2) (layer "B.Cu") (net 9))
 (segment (start 206.88 68.5) (end 188 68.5) (width 0.2) (layer "B.Cu") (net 9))
 (segment (start 214.92 76.54) (end 206.88 68.5) (width 0.2) (layer "B.Cu") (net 9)))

